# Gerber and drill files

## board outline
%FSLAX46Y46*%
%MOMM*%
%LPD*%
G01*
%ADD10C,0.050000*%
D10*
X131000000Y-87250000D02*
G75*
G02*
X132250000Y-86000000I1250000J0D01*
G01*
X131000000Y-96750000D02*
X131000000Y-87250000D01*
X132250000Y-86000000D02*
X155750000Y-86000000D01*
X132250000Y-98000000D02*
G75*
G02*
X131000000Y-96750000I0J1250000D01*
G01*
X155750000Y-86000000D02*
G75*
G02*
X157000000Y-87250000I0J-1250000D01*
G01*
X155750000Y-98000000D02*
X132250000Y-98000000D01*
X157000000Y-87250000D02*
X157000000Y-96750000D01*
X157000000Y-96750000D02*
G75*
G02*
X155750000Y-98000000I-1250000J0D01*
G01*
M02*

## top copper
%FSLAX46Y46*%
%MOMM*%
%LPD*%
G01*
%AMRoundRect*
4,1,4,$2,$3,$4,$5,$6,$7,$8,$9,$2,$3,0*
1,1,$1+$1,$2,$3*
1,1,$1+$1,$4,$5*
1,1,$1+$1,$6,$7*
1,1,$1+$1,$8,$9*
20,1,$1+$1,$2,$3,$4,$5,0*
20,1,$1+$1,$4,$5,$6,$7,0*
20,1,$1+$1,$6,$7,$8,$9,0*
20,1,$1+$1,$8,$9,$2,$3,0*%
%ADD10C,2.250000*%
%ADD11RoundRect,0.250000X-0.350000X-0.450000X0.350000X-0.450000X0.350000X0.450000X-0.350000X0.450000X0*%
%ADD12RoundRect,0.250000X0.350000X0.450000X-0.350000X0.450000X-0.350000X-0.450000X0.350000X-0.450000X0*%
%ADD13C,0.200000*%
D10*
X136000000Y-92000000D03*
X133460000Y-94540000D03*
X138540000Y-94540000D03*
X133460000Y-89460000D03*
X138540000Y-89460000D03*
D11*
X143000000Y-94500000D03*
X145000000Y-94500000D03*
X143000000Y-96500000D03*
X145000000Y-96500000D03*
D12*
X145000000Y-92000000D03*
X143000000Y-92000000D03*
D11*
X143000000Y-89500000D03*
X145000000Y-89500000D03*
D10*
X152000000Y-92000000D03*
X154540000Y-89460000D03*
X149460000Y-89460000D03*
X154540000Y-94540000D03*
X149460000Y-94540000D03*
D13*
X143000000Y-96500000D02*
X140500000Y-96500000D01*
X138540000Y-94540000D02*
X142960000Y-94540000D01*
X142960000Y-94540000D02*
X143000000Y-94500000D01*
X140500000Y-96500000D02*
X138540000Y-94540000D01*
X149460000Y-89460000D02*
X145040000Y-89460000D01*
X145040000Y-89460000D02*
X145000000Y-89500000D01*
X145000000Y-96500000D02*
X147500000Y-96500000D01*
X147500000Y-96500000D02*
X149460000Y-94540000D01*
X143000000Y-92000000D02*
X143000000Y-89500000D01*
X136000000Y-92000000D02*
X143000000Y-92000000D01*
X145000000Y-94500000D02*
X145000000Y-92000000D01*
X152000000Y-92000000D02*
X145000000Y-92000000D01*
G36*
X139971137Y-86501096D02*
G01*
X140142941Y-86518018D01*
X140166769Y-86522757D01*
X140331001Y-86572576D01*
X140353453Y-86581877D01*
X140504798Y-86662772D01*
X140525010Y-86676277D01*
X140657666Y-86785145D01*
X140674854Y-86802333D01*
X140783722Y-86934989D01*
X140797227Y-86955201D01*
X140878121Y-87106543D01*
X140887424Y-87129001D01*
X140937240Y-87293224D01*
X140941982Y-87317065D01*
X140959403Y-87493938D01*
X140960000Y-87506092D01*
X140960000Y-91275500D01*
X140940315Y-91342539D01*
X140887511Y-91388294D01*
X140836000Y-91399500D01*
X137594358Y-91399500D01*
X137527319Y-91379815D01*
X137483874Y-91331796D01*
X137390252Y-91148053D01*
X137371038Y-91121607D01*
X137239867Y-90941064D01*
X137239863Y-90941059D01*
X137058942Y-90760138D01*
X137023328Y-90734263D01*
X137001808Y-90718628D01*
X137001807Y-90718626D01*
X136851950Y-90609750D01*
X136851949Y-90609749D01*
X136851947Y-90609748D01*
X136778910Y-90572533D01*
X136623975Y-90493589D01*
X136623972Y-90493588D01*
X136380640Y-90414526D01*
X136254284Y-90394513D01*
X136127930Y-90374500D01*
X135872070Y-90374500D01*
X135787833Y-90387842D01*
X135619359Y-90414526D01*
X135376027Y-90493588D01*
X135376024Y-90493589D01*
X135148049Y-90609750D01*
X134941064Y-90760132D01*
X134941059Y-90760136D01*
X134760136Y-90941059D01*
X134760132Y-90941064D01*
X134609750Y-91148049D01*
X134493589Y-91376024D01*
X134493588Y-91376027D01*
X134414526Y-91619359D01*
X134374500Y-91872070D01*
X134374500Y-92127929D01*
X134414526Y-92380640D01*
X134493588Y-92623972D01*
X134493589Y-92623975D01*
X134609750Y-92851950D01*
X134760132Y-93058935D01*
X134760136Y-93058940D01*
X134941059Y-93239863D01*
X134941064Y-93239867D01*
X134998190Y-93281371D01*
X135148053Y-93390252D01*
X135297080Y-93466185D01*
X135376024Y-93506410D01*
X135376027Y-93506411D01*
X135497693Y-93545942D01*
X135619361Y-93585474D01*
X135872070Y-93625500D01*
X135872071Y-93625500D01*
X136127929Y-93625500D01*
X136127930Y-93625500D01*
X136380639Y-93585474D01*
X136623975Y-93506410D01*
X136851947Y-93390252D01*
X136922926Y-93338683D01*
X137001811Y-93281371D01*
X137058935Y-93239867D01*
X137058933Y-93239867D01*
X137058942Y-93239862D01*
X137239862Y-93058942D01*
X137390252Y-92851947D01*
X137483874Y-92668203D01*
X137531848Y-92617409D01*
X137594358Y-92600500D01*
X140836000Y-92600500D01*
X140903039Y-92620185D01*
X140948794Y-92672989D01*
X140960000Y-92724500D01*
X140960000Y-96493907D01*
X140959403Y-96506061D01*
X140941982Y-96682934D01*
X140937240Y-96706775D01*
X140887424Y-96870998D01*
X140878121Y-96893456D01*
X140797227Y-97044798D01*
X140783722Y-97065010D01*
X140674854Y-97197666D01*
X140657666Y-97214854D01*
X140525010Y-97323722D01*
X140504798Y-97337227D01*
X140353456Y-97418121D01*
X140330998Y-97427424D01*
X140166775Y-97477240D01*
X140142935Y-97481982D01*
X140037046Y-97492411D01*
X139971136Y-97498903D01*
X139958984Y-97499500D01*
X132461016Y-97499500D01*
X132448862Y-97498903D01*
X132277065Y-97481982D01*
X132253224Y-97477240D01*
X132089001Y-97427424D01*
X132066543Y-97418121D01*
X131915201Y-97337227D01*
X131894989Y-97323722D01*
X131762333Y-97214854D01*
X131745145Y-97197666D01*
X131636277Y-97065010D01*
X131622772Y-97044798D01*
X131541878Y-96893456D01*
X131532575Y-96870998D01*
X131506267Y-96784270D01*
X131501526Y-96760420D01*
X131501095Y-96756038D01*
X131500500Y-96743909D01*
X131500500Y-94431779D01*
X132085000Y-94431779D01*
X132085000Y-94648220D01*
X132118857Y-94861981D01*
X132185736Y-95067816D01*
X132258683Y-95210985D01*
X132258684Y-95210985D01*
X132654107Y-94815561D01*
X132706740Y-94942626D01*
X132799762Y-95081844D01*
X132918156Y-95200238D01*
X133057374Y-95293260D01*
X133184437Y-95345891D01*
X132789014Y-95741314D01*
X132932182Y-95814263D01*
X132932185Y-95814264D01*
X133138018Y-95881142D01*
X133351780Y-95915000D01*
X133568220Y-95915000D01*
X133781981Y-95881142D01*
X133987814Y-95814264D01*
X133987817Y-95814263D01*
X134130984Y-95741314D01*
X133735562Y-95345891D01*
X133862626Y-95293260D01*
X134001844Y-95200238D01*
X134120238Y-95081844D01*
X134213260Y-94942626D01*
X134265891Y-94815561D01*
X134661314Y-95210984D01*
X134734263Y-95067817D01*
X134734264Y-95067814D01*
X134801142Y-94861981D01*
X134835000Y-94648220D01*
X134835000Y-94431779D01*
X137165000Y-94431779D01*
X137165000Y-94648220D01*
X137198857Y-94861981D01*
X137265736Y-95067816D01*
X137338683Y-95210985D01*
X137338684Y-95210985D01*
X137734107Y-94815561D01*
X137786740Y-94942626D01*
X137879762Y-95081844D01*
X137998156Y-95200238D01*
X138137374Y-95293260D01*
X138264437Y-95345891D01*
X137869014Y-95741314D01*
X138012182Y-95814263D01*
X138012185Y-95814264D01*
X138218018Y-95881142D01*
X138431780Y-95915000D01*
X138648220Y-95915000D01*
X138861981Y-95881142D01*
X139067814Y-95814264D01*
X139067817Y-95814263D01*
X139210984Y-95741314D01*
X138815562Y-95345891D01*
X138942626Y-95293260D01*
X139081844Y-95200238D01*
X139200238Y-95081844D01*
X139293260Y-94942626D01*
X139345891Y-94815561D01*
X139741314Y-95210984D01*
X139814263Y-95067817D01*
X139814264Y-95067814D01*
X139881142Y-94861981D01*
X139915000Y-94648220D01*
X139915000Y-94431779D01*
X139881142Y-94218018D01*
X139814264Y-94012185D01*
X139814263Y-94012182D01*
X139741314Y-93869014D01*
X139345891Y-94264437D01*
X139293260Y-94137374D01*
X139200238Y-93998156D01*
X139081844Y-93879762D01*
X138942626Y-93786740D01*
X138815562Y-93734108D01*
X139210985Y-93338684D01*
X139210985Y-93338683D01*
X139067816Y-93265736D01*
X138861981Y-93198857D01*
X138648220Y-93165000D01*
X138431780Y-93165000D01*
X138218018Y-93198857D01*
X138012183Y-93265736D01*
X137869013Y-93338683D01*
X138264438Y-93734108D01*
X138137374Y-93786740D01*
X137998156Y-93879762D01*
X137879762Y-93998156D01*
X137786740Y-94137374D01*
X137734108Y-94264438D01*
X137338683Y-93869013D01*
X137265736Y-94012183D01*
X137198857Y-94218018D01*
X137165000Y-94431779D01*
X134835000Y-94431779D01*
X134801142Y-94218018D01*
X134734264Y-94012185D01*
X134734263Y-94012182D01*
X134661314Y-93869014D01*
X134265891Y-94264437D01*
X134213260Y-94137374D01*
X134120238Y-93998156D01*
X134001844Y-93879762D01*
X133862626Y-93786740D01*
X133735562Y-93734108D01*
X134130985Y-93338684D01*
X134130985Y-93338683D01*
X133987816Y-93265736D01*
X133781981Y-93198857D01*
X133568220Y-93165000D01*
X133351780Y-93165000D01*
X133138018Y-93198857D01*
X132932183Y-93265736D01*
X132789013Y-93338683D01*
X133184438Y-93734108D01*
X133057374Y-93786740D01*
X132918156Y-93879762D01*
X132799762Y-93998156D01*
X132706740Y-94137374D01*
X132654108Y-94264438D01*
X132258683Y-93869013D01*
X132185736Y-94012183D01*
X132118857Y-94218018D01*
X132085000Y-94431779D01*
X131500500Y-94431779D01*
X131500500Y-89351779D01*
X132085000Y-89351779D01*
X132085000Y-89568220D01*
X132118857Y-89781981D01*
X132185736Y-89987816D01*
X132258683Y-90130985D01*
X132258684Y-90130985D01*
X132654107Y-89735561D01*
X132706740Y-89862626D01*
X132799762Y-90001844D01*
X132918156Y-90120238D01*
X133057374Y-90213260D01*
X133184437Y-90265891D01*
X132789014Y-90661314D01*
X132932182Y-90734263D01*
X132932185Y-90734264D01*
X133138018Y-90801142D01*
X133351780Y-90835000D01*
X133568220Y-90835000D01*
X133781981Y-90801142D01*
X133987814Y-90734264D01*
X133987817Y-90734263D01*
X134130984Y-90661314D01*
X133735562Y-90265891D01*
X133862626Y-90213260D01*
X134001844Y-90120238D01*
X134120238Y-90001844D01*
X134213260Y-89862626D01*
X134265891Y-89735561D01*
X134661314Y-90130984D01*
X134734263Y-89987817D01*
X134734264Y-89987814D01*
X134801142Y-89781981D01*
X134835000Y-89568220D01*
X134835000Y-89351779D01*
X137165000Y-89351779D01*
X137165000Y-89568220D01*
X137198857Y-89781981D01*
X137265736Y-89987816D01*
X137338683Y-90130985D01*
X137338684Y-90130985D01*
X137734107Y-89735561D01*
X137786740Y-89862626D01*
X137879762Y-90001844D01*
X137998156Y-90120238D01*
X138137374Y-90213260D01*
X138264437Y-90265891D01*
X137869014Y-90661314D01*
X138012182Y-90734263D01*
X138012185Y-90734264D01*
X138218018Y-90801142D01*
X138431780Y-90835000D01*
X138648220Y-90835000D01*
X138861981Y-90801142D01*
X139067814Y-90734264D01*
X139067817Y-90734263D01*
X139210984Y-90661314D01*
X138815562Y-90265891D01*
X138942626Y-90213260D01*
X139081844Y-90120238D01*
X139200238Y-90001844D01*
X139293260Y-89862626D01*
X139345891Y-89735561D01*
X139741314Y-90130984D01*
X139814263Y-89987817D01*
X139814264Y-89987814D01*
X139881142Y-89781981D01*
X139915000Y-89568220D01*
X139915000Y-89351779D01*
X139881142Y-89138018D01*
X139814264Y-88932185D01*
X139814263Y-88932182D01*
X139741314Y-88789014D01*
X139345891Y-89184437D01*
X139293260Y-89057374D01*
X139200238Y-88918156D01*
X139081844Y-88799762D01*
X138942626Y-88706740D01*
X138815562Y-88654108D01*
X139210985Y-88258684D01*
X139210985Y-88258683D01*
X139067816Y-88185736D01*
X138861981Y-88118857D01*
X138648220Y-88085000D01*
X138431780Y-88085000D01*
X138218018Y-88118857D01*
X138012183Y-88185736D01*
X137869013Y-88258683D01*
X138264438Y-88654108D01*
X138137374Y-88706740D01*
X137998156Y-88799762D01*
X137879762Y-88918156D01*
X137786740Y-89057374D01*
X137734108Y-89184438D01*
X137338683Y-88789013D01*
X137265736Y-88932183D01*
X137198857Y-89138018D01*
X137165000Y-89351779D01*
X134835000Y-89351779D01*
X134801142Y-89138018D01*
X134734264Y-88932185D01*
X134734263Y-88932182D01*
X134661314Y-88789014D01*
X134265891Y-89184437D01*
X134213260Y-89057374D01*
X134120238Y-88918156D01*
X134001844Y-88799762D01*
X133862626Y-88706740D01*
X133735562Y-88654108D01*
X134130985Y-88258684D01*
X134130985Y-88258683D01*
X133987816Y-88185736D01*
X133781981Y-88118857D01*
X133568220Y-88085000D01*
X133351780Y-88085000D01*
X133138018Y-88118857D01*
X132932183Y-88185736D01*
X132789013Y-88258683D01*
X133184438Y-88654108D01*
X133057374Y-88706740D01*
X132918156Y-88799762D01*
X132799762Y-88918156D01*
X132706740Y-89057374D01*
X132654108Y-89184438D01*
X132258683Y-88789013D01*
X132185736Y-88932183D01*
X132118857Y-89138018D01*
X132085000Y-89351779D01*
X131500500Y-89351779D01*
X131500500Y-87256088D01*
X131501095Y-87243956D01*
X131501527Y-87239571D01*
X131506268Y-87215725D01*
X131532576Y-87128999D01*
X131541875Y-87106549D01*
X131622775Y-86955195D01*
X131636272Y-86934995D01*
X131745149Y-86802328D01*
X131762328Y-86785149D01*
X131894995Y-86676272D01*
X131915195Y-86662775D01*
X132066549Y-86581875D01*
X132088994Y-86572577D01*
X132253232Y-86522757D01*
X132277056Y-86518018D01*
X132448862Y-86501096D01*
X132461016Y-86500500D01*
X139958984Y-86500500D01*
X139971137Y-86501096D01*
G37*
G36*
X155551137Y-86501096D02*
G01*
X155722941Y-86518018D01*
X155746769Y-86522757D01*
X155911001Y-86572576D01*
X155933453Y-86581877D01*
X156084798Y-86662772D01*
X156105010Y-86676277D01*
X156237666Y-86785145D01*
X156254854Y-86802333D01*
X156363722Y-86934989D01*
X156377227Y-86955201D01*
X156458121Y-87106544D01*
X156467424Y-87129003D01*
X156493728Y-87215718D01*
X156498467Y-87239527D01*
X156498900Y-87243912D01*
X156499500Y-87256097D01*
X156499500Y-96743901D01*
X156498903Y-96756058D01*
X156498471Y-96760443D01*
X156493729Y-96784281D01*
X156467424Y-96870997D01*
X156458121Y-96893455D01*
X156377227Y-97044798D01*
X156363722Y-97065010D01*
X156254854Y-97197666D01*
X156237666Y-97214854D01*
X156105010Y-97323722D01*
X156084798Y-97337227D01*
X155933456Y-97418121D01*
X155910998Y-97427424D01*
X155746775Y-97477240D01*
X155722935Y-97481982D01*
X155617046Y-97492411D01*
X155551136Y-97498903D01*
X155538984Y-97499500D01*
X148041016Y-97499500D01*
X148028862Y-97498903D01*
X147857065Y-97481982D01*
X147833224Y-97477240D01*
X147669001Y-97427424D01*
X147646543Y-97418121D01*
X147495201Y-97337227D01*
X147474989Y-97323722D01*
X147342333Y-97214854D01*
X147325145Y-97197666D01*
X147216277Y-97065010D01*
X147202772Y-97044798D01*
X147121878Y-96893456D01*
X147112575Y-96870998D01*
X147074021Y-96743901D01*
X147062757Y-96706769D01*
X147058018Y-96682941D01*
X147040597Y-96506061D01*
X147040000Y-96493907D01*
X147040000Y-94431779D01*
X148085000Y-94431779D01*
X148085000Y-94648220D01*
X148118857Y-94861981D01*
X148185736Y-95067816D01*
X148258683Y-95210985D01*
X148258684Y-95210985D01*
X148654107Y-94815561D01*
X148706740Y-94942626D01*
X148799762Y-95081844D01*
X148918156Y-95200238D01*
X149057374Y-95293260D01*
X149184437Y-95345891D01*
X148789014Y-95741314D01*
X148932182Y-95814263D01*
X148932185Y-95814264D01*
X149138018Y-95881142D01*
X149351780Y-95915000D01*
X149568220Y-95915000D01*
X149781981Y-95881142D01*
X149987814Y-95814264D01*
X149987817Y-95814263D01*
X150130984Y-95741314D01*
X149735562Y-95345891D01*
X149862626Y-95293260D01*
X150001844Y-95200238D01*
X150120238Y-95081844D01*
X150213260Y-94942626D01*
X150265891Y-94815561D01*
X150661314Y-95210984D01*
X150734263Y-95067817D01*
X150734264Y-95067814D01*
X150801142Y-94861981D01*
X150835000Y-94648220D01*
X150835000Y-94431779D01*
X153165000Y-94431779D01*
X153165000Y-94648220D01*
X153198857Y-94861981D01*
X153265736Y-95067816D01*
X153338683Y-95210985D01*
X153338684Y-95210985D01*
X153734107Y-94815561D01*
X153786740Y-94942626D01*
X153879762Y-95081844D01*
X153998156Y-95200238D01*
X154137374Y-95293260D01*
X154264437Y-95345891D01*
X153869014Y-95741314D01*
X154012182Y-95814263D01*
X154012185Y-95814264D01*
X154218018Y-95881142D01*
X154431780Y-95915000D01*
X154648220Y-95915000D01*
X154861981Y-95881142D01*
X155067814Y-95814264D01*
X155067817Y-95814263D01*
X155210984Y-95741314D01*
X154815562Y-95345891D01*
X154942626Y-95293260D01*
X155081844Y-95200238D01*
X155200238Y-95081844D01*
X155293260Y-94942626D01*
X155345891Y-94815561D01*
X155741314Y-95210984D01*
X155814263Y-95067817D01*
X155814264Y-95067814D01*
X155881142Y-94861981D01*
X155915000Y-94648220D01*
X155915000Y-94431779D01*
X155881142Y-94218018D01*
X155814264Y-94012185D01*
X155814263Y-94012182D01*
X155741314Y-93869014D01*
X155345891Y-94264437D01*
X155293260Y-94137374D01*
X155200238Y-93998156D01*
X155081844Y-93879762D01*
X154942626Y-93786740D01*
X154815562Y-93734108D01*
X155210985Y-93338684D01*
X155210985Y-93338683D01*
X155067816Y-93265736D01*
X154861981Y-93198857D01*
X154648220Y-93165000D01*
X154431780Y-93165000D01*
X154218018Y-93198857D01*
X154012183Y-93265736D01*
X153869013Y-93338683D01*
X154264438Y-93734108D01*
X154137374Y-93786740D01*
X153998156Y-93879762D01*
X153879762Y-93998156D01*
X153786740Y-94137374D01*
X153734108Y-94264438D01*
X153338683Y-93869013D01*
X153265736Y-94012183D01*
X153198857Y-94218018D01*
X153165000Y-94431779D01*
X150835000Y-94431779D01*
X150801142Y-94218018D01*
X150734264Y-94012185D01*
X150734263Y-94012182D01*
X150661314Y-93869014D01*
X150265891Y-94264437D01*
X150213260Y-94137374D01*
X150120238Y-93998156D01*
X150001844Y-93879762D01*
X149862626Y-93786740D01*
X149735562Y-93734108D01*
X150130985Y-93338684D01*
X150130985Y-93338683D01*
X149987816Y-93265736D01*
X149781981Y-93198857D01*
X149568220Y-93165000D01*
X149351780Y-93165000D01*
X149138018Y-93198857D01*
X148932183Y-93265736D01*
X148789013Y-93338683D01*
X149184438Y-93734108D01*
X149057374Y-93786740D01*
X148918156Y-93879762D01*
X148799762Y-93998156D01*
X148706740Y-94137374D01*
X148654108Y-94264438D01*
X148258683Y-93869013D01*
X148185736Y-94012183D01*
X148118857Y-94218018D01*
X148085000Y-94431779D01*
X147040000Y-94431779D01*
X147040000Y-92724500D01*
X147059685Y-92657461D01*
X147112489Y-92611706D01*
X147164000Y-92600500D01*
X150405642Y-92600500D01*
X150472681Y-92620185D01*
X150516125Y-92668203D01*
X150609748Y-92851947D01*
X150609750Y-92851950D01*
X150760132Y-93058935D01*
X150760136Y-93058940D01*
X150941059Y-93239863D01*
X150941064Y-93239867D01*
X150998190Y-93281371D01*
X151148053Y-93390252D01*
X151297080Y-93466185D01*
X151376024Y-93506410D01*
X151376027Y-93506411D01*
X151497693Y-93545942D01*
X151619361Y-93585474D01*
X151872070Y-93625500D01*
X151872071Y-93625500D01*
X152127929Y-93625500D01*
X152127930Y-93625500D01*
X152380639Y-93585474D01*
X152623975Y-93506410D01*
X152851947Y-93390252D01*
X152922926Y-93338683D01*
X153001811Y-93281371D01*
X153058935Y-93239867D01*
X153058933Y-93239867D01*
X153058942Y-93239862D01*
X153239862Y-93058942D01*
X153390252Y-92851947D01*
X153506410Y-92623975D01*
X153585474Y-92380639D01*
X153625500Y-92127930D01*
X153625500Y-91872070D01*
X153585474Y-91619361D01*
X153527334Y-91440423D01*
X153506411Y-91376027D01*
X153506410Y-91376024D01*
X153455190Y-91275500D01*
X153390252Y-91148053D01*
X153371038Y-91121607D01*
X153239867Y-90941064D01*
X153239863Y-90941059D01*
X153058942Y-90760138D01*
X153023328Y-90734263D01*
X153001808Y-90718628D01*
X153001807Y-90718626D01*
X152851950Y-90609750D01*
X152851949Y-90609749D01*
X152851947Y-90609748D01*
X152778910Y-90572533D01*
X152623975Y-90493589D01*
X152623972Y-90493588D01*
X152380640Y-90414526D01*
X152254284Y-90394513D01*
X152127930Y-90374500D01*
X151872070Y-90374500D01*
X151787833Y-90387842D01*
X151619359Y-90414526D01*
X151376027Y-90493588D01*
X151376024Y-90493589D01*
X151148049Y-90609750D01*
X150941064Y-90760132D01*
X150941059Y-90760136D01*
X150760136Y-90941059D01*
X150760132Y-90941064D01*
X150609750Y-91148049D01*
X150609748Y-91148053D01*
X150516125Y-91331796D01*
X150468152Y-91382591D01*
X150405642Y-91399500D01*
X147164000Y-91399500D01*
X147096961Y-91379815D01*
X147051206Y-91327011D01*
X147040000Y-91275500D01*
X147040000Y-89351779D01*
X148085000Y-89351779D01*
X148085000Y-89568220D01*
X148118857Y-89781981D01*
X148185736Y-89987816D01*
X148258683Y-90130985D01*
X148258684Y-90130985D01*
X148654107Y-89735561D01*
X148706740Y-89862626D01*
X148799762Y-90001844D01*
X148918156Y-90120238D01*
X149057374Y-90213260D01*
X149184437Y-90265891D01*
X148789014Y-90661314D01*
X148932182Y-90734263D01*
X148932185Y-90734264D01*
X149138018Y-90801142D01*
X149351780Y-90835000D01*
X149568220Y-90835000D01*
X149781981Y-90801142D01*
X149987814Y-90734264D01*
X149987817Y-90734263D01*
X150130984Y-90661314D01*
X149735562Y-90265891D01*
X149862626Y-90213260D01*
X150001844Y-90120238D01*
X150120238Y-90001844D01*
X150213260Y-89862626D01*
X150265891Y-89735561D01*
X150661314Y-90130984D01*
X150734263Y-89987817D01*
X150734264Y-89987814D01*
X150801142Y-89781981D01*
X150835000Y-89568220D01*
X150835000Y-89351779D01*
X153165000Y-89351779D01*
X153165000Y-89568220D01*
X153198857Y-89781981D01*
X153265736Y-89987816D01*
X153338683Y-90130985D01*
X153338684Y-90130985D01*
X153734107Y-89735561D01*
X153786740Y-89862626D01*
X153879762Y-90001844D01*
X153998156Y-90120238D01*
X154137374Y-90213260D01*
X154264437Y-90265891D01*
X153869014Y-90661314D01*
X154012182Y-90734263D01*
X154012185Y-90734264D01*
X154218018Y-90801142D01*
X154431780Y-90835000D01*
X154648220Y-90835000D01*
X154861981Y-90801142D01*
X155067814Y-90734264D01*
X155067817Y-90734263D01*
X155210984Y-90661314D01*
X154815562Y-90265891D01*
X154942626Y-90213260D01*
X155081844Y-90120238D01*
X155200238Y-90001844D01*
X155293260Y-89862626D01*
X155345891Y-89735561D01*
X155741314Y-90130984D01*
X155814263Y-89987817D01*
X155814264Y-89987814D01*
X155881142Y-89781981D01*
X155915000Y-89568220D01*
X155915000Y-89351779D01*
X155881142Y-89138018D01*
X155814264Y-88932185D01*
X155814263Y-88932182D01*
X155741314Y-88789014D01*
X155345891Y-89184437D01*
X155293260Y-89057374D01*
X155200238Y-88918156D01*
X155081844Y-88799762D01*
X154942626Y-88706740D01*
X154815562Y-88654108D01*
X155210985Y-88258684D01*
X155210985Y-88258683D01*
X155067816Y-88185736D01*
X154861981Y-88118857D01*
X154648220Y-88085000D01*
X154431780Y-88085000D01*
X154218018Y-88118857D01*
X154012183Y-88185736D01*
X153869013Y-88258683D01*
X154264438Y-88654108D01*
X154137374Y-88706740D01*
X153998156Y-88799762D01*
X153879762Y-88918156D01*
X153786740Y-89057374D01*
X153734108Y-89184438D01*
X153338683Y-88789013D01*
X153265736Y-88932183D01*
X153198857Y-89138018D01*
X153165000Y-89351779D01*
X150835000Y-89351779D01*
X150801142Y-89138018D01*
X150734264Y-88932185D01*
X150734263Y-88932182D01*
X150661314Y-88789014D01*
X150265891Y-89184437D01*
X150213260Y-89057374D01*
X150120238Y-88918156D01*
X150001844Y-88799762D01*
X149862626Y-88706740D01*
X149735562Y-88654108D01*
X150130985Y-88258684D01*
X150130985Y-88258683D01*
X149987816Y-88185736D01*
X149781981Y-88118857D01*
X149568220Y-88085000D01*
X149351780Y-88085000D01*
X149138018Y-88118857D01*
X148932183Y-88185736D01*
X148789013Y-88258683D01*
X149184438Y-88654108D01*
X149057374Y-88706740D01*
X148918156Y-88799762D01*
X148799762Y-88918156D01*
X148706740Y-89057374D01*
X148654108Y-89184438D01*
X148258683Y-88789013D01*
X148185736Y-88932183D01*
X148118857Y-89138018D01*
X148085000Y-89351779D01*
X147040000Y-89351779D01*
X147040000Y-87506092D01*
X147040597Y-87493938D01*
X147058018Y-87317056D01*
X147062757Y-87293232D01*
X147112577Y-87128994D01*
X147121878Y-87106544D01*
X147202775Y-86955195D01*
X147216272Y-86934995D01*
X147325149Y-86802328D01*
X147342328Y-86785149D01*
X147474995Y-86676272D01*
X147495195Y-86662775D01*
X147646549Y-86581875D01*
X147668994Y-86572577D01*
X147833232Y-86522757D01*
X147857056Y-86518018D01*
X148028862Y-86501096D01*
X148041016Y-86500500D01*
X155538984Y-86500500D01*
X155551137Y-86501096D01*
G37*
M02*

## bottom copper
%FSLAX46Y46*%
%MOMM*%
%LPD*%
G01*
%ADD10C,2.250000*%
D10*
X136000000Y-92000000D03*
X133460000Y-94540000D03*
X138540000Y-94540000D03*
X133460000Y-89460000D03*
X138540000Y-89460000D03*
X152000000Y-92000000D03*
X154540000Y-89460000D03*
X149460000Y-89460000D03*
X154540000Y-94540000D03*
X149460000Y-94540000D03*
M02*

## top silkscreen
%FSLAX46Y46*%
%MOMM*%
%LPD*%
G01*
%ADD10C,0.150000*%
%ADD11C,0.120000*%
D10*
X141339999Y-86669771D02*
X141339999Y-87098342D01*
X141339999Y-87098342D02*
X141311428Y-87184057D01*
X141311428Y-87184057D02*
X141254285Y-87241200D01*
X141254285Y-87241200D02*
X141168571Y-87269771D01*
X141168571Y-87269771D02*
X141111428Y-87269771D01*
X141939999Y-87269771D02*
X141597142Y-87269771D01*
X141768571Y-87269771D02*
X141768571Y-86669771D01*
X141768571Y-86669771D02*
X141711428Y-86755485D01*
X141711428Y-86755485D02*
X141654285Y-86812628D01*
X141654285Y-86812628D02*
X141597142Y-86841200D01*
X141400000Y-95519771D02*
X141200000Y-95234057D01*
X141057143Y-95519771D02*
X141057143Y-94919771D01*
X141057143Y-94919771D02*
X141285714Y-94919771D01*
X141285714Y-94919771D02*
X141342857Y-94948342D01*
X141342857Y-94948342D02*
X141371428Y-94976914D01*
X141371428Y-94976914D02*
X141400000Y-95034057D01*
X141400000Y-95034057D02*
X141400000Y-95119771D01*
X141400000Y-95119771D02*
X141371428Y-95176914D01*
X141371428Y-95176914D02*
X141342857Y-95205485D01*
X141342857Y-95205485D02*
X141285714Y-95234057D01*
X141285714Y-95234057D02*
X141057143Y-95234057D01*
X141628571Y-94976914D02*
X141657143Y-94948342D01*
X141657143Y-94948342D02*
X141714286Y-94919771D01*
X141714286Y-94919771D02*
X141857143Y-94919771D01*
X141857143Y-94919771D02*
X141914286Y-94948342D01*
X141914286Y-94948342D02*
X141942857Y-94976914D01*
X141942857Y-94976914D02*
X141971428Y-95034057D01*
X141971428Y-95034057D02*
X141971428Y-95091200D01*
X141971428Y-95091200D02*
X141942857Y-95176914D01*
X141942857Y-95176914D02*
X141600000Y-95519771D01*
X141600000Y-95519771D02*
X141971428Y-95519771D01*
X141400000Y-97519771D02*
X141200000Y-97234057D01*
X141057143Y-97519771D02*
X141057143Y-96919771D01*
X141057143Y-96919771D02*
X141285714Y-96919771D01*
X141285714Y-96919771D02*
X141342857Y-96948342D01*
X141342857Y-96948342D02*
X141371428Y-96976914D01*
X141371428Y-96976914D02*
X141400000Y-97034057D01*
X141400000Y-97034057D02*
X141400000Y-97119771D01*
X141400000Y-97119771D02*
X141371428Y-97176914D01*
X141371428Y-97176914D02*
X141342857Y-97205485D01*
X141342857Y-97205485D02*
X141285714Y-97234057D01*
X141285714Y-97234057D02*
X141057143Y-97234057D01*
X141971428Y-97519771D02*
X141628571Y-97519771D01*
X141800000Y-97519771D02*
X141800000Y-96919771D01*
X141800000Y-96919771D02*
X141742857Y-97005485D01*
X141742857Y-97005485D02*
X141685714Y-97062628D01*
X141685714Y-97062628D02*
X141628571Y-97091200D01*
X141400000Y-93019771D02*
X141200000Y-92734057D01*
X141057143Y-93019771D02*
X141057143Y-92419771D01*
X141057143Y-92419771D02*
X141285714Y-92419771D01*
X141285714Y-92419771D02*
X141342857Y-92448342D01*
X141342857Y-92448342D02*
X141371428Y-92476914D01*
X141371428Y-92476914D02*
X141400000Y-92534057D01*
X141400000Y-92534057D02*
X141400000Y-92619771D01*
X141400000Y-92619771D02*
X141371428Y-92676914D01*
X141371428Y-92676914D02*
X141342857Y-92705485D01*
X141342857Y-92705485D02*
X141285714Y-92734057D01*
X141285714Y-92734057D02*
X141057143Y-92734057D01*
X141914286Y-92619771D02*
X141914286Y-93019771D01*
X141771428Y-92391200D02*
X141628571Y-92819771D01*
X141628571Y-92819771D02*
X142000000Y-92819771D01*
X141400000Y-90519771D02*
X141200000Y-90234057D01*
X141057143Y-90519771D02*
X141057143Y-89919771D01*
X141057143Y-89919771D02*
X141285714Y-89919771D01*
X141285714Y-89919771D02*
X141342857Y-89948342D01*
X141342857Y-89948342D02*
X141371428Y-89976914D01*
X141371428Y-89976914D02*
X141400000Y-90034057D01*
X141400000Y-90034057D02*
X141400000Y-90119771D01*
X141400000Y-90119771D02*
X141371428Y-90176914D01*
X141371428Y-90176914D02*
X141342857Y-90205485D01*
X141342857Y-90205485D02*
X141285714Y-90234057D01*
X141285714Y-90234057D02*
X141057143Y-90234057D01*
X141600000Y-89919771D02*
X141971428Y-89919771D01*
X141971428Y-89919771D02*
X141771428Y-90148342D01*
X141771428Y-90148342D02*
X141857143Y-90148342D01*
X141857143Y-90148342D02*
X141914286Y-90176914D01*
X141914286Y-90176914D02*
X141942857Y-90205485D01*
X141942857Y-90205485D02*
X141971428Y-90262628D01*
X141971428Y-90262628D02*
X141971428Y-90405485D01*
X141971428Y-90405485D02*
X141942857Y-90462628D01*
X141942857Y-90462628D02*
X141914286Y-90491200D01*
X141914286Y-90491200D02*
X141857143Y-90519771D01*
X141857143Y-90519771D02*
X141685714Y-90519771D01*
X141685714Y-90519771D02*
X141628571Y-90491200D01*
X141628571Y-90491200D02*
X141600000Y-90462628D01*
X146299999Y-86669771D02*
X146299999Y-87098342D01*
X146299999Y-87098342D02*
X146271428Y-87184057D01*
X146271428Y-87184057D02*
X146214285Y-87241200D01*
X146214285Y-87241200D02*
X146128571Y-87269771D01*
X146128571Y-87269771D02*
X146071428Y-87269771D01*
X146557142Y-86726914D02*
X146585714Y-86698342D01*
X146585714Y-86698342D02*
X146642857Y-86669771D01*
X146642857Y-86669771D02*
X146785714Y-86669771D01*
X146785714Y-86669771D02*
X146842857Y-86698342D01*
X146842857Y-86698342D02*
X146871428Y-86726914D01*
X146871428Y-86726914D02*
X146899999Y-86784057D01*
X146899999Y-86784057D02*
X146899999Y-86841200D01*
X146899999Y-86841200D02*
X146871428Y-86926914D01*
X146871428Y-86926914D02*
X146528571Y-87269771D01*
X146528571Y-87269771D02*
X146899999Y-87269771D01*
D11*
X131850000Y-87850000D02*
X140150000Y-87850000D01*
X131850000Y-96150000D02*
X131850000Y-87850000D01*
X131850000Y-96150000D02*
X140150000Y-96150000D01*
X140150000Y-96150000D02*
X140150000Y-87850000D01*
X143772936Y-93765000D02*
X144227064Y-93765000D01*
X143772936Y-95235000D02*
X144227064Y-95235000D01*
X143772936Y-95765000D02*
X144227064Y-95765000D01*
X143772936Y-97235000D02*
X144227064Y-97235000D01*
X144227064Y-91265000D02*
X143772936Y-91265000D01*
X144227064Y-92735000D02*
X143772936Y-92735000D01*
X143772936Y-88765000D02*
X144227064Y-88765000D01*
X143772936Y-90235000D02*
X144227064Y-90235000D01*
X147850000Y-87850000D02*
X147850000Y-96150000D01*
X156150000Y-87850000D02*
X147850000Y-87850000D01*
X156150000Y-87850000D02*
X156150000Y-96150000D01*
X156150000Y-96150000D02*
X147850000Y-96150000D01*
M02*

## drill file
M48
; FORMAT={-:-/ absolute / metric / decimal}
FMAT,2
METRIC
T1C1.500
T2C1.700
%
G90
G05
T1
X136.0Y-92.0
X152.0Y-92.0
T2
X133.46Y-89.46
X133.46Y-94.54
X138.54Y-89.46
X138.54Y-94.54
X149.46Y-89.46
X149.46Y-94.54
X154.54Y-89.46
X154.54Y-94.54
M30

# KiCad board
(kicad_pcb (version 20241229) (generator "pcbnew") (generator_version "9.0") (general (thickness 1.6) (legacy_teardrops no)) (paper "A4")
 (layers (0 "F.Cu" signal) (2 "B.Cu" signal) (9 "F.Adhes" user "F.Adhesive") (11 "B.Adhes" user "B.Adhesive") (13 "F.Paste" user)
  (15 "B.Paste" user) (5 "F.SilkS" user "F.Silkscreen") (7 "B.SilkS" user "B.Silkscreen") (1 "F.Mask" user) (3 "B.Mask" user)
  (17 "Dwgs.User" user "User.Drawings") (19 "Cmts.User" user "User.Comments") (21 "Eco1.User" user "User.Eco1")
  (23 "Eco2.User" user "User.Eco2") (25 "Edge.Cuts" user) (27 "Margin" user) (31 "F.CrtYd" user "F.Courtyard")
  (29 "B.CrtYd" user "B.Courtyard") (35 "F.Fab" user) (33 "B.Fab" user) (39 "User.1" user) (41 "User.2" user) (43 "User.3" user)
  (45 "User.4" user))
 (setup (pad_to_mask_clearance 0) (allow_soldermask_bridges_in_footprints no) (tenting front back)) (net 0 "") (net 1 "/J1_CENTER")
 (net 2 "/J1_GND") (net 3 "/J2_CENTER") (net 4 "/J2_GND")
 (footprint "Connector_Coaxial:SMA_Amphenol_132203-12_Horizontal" (layer "F.Cu") (at 136 92 90)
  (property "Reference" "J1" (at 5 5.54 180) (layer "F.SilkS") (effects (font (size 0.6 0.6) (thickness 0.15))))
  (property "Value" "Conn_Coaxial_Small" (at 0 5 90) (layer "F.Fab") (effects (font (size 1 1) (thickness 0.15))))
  (fp_line (start 4.15 -4.15) (end 4.15 4.15) (stroke (width 0.12) (type solid)) (layer "F.SilkS"))
  (fp_line (start -4.15 -4.15) (end 4.15 -4.15) (stroke (width 0.12) (type solid)) (layer "F.SilkS"))
  (fp_line (start -4.15 -4.15) (end -4.15 4.15) (stroke (width 0.12) (type solid)) (layer "F.SilkS"))
  (fp_line (start -4.15 4.15) (end 4.15 4.15) (stroke (width 0.12) (type solid)) (layer "F.SilkS"))
  (pad "1" thru_hole circle (at 0 0 90) (size 2.25 2.25) (drill 1.5) (layers "*.Cu" "*.Mask") (remove_unused_layers no) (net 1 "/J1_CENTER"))
  (pad "2" thru_hole circle (at -2.54 -2.54 90) (size 2.25 2.25) (drill 1.7) (layers "*.Cu" "*.Mask") (remove_unused_layers no)
   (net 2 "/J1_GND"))
  (pad "2" thru_hole circle (at -2.54 2.54 90) (size 2.25 2.25) (drill 1.7) (layers "*.Cu" "*.Mask") (remove_unused_layers no)
   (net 2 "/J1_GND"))
  (pad "2" thru_hole circle (at 2.54 -2.54 90) (size 2.25 2.25) (drill 1.7) (layers "*.Cu" "*.Mask") (remove_unused_layers no)
   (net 2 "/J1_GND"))
  (pad "2" thru_hole circle (at 2.54 2.54 180) (size 2.25 2.25) (drill 1.7) (layers "*.Cu" "*.Mask") (remove_unused_layers no)
   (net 2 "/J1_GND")))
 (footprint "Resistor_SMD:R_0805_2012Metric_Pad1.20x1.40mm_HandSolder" (layer "F.Cu") (at 144 94.5)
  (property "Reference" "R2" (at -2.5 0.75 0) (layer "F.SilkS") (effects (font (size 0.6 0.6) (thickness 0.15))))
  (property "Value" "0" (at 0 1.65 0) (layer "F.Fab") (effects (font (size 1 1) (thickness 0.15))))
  (fp_line (start -0.227064 -0.735) (end 0.227064 -0.735) (stroke (width 0.12) (type solid)) (layer "F.SilkS"))
  (fp_line (start -0.227064 0.735) (end 0.227064 0.735) (stroke (width 0.12) (type solid)) (layer "F.SilkS"))
  (pad "1" smd roundrect (at -1 0) (size 1.2 1.4) (layers "F.Cu" "F.Mask" "F.Paste") (roundrect_rratio 0.208333) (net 2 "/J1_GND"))
  (pad "2" smd roundrect (at 1 0) (size 1.2 1.4) (layers "F.Cu" "F.Mask" "F.Paste") (roundrect_rratio 0.208333) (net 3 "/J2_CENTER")))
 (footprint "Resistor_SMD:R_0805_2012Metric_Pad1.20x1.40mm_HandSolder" (layer "F.Cu") (at 144 96.5)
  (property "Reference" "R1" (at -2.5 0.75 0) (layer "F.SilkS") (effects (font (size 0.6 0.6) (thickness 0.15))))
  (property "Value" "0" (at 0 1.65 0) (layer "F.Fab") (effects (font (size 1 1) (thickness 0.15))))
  (fp_line (start -0.227064 -0.735) (end 0.227064 -0.735) (stroke (width 0.12) (type solid)) (layer "F.SilkS"))
  (fp_line (start -0.227064 0.735) (end 0.227064 0.735) (stroke (width 0.12) (type solid)) (layer "F.SilkS"))
  (pad "1" smd roundrect (at -1 0) (size 1.2 1.4) (layers "F.Cu" "F.Mask" "F.Paste") (roundrect_rratio 0.208333) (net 2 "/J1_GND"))
  (pad "2" smd roundrect (at 1 0) (size 1.2 1.4) (layers "F.Cu" "F.Mask" "F.Paste") (roundrect_rratio 0.208333) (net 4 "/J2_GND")))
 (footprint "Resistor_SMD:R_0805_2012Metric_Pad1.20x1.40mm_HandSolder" (layer "F.Cu") (at 144 92 180)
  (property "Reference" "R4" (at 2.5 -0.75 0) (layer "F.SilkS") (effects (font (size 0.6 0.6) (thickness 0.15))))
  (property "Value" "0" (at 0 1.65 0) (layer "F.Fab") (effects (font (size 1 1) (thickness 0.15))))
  (fp_line (start -0.227064 0.735) (end 0.227064 0.735) (stroke (width 0.12) (type solid)) (layer "F.SilkS"))
  (fp_line (start -0.227064 -0.735) (end 0.227064 -0.735) (stroke (width 0.12) (type solid)) (layer "F.SilkS"))
  (pad "1" smd roundrect (at -1 0 180) (size 1.2 1.4) (layers "F.Cu" "F.Mask" "F.Paste") (roundrect_rratio 0.208333) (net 3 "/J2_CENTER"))
  (pad "2" smd roundrect (at 1 0 180) (size 1.2 1.4) (layers "F.Cu" "F.Mask" "F.Paste") (roundrect_rratio 0.208333) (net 1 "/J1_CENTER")))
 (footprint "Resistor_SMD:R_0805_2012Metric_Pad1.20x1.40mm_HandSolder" (layer "F.Cu") (at 144 89.5)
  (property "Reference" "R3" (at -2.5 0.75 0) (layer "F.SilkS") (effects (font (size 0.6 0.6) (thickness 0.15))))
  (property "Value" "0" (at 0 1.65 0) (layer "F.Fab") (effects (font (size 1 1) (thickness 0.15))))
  (fp_line (start -0.227064 -0.735) (end 0.227064 -0.735) (stroke (width 0.12) (type solid)) (layer "F.SilkS"))
  (fp_line (start -0.227064 0.735) (end 0.227064 0.735) (stroke (width 0.12) (type solid)) (layer "F.SilkS"))
  (pad "1" smd roundrect (at -1 0) (size 1.2 1.4) (layers "F.Cu" "F.Mask" "F.Paste") (roundrect_rratio 0.208333) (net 1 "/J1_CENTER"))
  (pad "2" smd roundrect (at 1 0) (size 1.2 1.4) (layers "F.Cu" "F.Mask" "F.Paste") (roundrect_rratio 0.208333) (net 4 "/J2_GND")))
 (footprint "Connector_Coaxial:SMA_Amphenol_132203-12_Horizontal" (layer "F.Cu") (at 152 92 -90)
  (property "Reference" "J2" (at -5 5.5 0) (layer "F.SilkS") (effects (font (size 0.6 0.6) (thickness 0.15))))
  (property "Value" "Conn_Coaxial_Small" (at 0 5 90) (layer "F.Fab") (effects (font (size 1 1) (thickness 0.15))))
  (fp_line (start -4.15 4.15) (end 4.15 4.15) (stroke (width 0.12) (type solid)) (layer "F.SilkS"))
  (fp_line (start -4.15 -4.15) (end -4.15 4.15) (stroke (width 0.12) (type solid)) (layer "F.SilkS"))
  (fp_line (start -4.15 -4.15) (end 4.15 -4.15) (stroke (width 0.12) (type solid)) (layer "F.SilkS"))
  (fp_line (start 4.15 -4.15) (end 4.15 4.15) (stroke (width 0.12) (type solid)) (layer "F.SilkS"))
  (pad "1" thru_hole circle (at 0 0 270) (size 2.25 2.25) (drill 1.5) (layers "*.Cu" "*.Mask") (remove_unused_layers no)
   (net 3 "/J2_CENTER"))
  (pad "2" thru_hole circle (at -2.54 -2.54 270) (size 2.25 2.25) (drill 1.7) (layers "*.Cu" "*.Mask") (remove_unused_layers no)
   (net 4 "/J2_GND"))
  (pad "2" thru_hole circle (at -2.54 2.54 270) (size 2.25 2.25) (drill 1.7) (layers "*.Cu" "*.Mask") (remove_unused_layers no)
   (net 4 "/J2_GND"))
  (pad "2" thru_hole circle (at 2.54 -2.54 270) (size 2.25 2.25) (drill 1.7) (layers "*.Cu" "*.Mask") (remove_unused_layers no)
   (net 4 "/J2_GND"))
  (pad "2" thru_hole circle (at 2.54 2.54) (size 2.25 2.25) (drill 1.7) (layers "*.Cu" "*.Mask") (remove_unused_layers no) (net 4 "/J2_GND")))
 (gr_arc (start 131 87.25) (mid 131.366117 86.366117) (end 132.25 86) (stroke (width 0.05) (type default)) (layer "Edge.Cuts"))
 (gr_line (start 131 96.75) (end 131 87.25) (stroke (width 0.05) (type default)) (layer "Edge.Cuts"))
 (gr_line (start 132.25 86) (end 155.75 86) (stroke (width 0.05) (type default)) (layer "Edge.Cuts"))
 (gr_arc (start 132.25 98) (mid 131.366117 97.633883) (end 131 96.75) (stroke (width 0.05) (type default)) (layer "Edge.Cuts"))
 (gr_arc (start 155.75 86) (mid 156.633883 86.366117) (end 157 87.25) (stroke (width 0.05) (type default)) (layer "Edge.Cuts"))
 (gr_line (start 155.75 98) (end 132.25 98) (stroke (width 0.05) (type default)) (layer "Edge.Cuts"))
 (gr_line (start 157 87.25) (end 157 96.75) (stroke (width 0.05) (type default)) (layer "Edge.Cuts"))
 (gr_arc (start 157 96.75) (mid 156.633883 97.633883) (end 155.75 98) (stroke (width 0.05) (type default)) (layer "Edge.Cuts"))
 (segment (start 143 96.5) (end 140.5 96.5) (width 0.2) (layer "F.Cu") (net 2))
 (segment (start 138.54 94.54) (end 142.96 94.54) (width 0.2) (layer "F.Cu") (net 2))
 (segment (start 142.96 94.54) (end 143 94.5) (width 0.2) (layer "F.Cu") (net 2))
 (segment (start 140.5 96.5) (end 138.54 94.54) (width 0.2) (layer "F.Cu") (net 2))
 (segment (start 149.46 89.46) (end 145.04 89.46) (width 0.2) (layer "F.Cu") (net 4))
 (segment (start 145.04 89.46) (end 145 89.5) (width 0.2) (layer "F.Cu") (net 4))
 (segment (start 145 96.5) (end 147.5 96.5) (width 0.2) (layer "F.Cu") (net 4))
 (segment (start 147.5 96.5) (end 149.46 94.54) (width 0.2) (layer "F.Cu") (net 4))
 (segment (start 143 92) (end 143 89.5) (width 0.2) (layer "F.Cu") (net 1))
 (segment (start 136 92) (end 143 92) (width 0.2) (layer "F.Cu") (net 1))
 (segment (start 145 94.5) (end 145 92) (width 0.2) (layer "F.Cu") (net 3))
 (segment (start 152 92) (end 145 92) (width 0.2) (layer "F.Cu") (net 3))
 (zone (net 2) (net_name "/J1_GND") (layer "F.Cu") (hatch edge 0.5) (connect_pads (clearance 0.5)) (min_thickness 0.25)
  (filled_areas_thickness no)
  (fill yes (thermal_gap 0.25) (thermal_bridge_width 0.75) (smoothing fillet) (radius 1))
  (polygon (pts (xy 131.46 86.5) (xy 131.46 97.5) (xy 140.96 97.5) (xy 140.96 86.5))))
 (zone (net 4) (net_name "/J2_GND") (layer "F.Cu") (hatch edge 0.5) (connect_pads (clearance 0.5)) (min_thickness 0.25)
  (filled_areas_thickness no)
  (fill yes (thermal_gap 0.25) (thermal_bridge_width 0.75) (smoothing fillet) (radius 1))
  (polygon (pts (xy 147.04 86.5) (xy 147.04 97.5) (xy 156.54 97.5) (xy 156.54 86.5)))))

